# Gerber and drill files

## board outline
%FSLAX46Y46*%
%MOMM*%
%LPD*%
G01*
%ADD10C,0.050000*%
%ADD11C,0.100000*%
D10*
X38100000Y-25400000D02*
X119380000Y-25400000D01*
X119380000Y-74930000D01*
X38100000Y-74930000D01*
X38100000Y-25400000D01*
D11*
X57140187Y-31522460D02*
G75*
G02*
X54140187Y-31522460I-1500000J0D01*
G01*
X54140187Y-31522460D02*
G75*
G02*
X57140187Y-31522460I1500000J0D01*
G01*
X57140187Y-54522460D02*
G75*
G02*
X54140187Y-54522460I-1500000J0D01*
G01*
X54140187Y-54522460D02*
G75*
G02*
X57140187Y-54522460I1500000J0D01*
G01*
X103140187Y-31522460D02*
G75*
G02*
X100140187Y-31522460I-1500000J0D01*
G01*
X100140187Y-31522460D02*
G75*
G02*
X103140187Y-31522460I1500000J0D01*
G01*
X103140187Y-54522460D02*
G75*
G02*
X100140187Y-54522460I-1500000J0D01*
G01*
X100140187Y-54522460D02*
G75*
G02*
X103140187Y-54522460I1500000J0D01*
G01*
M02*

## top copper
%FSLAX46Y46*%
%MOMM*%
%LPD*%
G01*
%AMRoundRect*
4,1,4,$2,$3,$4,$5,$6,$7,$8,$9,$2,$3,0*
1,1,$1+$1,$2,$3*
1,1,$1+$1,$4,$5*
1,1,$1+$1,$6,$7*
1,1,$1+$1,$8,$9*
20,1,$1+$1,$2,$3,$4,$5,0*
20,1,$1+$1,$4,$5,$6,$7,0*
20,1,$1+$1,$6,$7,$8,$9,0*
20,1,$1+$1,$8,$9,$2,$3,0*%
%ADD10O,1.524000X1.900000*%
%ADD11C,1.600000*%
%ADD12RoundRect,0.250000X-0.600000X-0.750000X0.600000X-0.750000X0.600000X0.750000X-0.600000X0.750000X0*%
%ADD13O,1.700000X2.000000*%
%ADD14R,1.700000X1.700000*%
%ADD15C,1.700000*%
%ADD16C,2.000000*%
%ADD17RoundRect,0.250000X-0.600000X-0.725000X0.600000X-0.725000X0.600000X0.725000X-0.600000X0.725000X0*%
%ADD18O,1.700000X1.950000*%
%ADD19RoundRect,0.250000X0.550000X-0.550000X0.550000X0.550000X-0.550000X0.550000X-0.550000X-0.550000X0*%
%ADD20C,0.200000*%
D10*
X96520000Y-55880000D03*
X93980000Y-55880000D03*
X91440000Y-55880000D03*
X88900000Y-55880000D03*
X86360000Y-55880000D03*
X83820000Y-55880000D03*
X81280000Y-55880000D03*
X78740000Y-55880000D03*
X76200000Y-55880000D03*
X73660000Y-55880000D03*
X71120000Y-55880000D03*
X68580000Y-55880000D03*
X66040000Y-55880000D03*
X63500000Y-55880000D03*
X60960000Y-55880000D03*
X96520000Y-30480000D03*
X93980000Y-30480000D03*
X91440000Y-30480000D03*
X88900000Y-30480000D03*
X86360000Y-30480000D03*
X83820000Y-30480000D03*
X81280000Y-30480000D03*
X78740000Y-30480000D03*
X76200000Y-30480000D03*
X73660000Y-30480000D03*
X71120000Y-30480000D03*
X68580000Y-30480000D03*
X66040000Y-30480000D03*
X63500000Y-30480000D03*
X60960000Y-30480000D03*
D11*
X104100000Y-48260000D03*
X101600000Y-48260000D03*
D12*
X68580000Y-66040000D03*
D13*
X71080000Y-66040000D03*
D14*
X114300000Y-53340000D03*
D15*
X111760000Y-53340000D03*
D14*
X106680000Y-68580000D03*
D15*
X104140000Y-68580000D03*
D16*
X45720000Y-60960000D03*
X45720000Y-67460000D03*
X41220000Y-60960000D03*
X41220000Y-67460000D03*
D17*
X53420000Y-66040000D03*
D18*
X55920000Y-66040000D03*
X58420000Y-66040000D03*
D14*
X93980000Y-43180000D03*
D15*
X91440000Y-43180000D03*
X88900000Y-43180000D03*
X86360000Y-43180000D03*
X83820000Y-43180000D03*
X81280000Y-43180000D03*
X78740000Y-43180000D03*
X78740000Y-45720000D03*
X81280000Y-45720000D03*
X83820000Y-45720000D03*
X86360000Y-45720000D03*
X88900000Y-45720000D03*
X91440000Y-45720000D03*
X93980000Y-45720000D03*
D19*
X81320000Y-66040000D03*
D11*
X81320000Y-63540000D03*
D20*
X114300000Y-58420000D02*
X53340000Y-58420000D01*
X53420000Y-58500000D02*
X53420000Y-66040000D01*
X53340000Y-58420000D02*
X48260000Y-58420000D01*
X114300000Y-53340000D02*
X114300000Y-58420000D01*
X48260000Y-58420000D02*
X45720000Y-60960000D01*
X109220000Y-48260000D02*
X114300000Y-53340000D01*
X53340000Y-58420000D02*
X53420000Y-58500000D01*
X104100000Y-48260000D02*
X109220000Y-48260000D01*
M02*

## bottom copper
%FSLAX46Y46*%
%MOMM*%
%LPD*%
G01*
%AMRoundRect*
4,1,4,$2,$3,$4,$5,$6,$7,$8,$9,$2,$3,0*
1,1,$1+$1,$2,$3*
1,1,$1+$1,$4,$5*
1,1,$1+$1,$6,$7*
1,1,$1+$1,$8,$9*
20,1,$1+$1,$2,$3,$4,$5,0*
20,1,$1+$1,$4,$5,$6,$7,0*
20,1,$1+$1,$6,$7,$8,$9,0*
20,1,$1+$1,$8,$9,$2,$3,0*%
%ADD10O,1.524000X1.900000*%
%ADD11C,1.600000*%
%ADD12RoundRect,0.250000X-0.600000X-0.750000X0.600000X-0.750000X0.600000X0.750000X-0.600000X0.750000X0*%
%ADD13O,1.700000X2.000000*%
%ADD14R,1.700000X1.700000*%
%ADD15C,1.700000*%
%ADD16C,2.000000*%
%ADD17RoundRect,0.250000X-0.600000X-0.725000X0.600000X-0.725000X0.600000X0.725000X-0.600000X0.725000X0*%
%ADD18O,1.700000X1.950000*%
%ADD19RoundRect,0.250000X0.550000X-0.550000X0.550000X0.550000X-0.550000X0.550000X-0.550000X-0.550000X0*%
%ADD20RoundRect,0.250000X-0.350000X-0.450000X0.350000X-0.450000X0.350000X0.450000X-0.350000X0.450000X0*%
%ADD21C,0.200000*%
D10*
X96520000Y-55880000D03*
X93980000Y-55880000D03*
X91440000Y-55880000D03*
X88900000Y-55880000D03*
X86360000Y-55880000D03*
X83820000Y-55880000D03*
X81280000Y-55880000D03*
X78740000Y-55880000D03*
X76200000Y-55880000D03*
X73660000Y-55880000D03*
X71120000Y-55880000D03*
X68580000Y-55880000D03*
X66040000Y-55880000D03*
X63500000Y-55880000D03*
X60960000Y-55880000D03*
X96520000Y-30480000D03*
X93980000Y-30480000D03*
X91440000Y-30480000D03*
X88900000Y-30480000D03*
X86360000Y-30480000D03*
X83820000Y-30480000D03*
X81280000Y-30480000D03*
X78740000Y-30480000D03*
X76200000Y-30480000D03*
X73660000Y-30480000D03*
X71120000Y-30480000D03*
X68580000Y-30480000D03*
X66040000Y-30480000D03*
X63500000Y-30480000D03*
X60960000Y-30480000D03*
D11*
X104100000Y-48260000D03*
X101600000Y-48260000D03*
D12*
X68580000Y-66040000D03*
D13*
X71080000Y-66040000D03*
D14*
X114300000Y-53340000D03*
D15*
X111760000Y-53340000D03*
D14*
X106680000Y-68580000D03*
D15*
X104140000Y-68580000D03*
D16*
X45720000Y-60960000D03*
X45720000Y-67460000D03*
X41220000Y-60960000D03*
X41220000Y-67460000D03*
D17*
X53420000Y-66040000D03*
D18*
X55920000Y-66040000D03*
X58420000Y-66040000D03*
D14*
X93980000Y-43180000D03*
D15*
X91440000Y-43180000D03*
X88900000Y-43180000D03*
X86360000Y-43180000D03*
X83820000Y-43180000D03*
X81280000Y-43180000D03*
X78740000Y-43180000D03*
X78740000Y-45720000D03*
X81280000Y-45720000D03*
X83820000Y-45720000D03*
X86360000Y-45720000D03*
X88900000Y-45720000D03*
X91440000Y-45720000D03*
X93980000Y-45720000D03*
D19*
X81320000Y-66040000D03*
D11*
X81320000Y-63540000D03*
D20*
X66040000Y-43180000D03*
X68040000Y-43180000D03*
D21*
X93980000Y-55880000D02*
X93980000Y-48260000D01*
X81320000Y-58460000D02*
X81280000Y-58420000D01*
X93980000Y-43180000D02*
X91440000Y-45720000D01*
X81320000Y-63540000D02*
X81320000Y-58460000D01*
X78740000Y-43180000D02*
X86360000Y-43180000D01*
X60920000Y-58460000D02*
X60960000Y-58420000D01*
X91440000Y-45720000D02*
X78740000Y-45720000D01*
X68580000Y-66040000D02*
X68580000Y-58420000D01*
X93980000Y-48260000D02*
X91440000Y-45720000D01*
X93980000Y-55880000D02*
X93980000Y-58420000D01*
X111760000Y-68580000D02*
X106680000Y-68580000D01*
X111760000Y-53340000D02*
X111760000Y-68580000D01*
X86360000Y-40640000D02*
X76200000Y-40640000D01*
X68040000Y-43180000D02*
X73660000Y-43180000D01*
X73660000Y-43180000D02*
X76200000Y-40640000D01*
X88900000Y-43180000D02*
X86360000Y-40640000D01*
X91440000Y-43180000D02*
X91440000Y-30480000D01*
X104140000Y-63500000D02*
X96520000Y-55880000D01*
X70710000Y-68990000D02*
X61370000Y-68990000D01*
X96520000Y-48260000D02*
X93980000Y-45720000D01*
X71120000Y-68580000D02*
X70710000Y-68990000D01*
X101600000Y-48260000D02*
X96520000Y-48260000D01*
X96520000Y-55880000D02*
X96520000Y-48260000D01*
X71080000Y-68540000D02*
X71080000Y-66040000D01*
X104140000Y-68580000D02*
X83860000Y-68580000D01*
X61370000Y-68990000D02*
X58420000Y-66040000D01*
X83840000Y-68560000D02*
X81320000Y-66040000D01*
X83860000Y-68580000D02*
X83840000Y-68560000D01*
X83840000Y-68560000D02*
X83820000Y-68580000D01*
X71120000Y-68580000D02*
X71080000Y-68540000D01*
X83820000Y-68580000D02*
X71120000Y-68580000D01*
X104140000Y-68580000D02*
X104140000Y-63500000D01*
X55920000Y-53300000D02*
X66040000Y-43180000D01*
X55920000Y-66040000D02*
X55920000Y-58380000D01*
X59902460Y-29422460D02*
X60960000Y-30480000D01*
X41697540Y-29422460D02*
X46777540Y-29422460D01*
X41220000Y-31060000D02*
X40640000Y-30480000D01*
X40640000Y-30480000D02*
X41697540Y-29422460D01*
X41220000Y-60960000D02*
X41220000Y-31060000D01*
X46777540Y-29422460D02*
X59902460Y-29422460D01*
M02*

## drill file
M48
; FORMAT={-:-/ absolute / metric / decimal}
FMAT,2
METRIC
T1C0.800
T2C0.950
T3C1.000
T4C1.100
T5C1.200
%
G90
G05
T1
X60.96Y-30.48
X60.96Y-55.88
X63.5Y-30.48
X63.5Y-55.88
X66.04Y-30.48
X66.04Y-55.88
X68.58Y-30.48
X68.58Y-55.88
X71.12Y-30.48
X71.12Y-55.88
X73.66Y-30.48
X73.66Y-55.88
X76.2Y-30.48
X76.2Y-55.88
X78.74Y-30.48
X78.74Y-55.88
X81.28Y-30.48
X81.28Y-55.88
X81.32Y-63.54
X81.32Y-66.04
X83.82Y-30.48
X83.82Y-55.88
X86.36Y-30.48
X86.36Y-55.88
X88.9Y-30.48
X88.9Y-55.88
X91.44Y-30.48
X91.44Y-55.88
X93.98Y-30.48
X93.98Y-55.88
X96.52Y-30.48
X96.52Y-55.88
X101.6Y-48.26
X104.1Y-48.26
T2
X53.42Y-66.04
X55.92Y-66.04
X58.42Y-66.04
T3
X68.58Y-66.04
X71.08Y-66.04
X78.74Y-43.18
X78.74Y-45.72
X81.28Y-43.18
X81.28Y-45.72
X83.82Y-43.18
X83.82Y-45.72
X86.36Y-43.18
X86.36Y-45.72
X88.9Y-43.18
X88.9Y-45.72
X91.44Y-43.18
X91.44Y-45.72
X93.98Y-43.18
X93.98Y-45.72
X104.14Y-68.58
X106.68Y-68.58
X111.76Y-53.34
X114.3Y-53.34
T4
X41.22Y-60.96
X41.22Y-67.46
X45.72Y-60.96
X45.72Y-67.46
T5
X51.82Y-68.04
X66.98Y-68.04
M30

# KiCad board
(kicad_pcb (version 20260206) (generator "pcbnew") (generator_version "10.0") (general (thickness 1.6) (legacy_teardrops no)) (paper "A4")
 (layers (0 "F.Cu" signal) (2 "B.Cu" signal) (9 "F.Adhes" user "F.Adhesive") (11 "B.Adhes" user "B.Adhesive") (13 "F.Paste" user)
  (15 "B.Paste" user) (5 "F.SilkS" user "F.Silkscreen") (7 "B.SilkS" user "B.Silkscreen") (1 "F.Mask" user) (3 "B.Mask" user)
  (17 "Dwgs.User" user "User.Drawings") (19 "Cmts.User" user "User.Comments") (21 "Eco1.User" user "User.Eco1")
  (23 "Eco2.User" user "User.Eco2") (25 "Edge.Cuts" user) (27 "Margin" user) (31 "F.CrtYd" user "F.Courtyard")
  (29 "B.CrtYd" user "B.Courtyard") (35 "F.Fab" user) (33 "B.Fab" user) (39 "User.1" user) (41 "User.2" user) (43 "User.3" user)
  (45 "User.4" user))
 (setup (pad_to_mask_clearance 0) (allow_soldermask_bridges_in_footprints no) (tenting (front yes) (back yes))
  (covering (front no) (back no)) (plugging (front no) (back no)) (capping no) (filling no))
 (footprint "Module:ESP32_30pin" (layer "F.Cu") (at 79.500187 43.95246 90)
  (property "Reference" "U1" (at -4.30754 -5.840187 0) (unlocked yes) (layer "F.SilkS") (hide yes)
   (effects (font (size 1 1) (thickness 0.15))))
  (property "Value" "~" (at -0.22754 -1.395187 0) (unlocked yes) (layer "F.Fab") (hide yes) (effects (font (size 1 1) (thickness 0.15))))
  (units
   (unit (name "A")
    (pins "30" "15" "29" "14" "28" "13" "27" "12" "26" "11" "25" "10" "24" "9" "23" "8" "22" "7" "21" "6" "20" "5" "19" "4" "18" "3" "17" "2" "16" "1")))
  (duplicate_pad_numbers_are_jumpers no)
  (fp_circle (center 12.43 -23.86) (end 12.43 -22.36) (stroke (width 0.1) (type default)) (fill no) (layer "Edge.Cuts"))
  (fp_circle (center -10.57 -23.86) (end -10.57 -22.36) (stroke (width 0.1) (type default)) (fill no) (layer "Edge.Cuts"))
  (fp_circle (center 12.43 22.14) (end 12.43 23.64) (stroke (width 0.1) (type default)) (fill no) (layer "Edge.Cuts"))
  (fp_circle (center -10.57 22.14) (end -10.57 23.64) (stroke (width 0.1) (type default)) (fill no) (layer "Edge.Cuts"))
  (pad "1" thru_hole oval (at -11.92754 17.019813) (size 1.524 1.9) (drill 0.8) (layers "*.Cu" "*.Mask") (remove_unused_layers no)
   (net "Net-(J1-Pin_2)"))
  (pad "2" thru_hole oval (at -11.92754 14.479813) (size 1.524 1.9) (drill 0.8) (layers "*.Cu" "*.Mask") (remove_unused_layers no)
   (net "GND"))
  (pad "3" thru_hole oval (at -11.92754 11.939813) (size 1.524 1.9) (drill 0.8) (layers "*.Cu" "*.Mask") (remove_unused_layers no)
   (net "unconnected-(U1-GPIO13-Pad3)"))
  (pad "4" thru_hole oval (at -11.92754 9.399813) (size 1.524 1.9) (drill 0.8) (layers "*.Cu" "*.Mask") (remove_unused_layers no)
   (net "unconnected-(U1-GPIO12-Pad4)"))
  (pad "5" thru_hole oval (at -11.92754 6.859813) (size 1.524 1.9) (drill 0.8) (layers "*.Cu" "*.Mask") (remove_unused_layers no)
   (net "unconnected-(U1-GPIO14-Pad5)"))
  (pad "6" thru_hole oval (at -11.92754 4.319813) (size 1.524 1.9) (drill 0.8) (layers "*.Cu" "*.Mask") (remove_unused_layers no)
   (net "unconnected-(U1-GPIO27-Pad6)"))
  (pad "7" thru_hole oval (at -11.92754 1.779813) (size 1.524 1.9) (drill 0.8) (layers "*.Cu" "*.Mask") (remove_unused_layers no)
   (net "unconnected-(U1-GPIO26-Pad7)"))
  (pad "8" thru_hole oval (at -11.92754 -0.760187) (size 1.524 1.9) (drill 0.8) (layers "*.Cu" "*.Mask") (remove_unused_layers no)
   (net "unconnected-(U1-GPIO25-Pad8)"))
  (pad "9" thru_hole oval (at -11.92754 -3.300187) (size 1.524 1.9) (drill 0.8) (layers "*.Cu" "*.Mask") (remove_unused_layers no)
   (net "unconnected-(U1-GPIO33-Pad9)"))
  (pad "10" thru_hole oval (at -11.92754 -5.840187) (size 1.524 1.9) (drill 0.8) (layers "*.Cu" "*.Mask") (remove_unused_layers no)
   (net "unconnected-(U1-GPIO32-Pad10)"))
  (pad "11" thru_hole oval (at -11.92754 -8.380187) (size 1.524 1.9) (drill 0.8) (layers "*.Cu" "*.Mask") (remove_unused_layers no)
   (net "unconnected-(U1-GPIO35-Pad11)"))
  (pad "12" thru_hole oval (at -11.92754 -10.920187) (size 1.524 1.9) (drill 0.8) (layers "*.Cu" "*.Mask") (remove_unused_layers no)
   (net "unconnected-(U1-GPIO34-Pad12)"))
  (pad "13" thru_hole oval (at -11.92754 -13.460187) (size 1.524 1.9) (drill 0.8) (layers "*.Cu" "*.Mask") (remove_unused_layers no)
   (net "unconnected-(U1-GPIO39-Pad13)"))
  (pad "14" thru_hole oval (at -11.92754 -16.000187) (size 1.524 1.9) (drill 0.8) (layers "*.Cu" "*.Mask") (remove_unused_layers no)
   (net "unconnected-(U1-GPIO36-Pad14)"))
  (pad "15" thru_hole oval (at -11.92754 -18.540187) (size 1.524 1.9) (drill 0.8) (layers "*.Cu" "*.Mask") (remove_unused_layers no)
   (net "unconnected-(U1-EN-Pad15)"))
  (pad "16" thru_hole oval (at 13.47246 17.019813) (size 1.524 1.9) (drill 0.8) (layers "*.Cu" "*.Mask") (remove_unused_layers no)
   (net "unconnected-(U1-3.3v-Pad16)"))
  (pad "17" thru_hole oval (at 13.47246 14.479813) (size 1.524 1.9) (drill 0.8) (layers "*.Cu" "*.Mask") (remove_unused_layers no)
   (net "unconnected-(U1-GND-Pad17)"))
  (pad "18" thru_hole oval (at 13.47246 11.939813) (size 1.524 1.9) (drill 0.8) (layers "*.Cu" "*.Mask") (remove_unused_layers no)
   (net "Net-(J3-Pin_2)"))
  (pad "19" thru_hole oval (at 13.47246 9.399813) (size 1.524 1.9) (drill 0.8) (layers "*.Cu" "*.Mask") (remove_unused_layers no)
   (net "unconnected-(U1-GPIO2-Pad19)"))
  (pad "20" thru_hole oval (at 13.47246 6.859813) (size 1.524 1.9) (drill 0.8) (layers "*.Cu" "*.Mask" "Dwgs.User")
   (remove_unused_layers no) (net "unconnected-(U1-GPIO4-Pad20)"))
  (pad "21" thru_hole oval (at 13.47246 4.319813) (size 1.524 1.9) (drill 0.8) (layers "*.Cu" "*.Mask") (remove_unused_layers no)
   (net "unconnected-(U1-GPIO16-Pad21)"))
  (pad "22" thru_hole oval (at 13.47246 1.779813) (size 1.524 1.9) (drill 0.8) (layers "*.Cu" "*.Mask") (remove_unused_layers no)
   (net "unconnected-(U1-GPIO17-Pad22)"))
  (pad "23" thru_hole oval (at 13.47246 -0.760187) (size 1.524 1.9) (drill 0.8) (layers "*.Cu" "*.Mask") (remove_unused_layers no)
   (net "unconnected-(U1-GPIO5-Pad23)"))
  (pad "24" thru_hole oval (at 13.47246 -3.300187) (size 1.524 1.9) (drill 0.8) (layers "*.Cu" "*.Mask") (remove_unused_layers no)
   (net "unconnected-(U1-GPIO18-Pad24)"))
  (pad "25" thru_hole oval (at 13.47246 -5.840187) (size 1.524 1.9) (drill 0.8) (layers "*.Cu" "*.Mask") (remove_unused_layers no)
   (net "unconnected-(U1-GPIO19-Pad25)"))
  (pad "26" thru_hole oval (at 13.47246 -8.380187) (size 1.524 1.9) (drill 0.8) (layers "*.Cu" "*.Mask") (remove_unused_layers no)
   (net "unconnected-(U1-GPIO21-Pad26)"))
  (pad "27" thru_hole oval (at 13.47246 -10.920187) (size 1.524 1.9) (drill 0.8) (layers "*.Cu" "*.Mask") (remove_unused_layers no)
   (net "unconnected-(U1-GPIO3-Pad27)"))
  (pad "28" thru_hole oval (at 13.47246 -13.460187) (size 1.524 1.9) (drill 0.8) (layers "*.Cu" "*.Mask") (remove_unused_layers no)
   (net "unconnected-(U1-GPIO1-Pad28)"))
  (pad "29" thru_hole oval (at 13.47246 -16.000187) (size 1.524 1.9) (drill 0.8) (layers "*.Cu" "*.Mask") (remove_unused_layers no)
   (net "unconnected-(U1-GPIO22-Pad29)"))
  (pad "30" thru_hole oval (at 13.47246 -18.540187) (size 1.524 1.9) (drill 0.8) (layers "*.Cu" "*.Mask") (remove_unused_layers no)
   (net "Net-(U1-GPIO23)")))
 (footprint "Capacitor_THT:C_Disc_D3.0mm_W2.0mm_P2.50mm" (layer "F.Cu") (at 104.1 48.26 180)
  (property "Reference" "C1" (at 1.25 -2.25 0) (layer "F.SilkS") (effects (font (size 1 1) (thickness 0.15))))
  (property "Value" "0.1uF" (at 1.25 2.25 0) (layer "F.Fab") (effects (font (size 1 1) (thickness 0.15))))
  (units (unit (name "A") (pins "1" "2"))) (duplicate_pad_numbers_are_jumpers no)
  (pad "1" thru_hole circle (at 0 0 180) (size 1.6 1.6) (drill 0.8) (layers "*.Cu" "*.Mask") (remove_unused_layers no) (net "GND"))
  (pad "2" thru_hole circle (at 2.5 0 180) (size 1.6 1.6) (drill 0.8) (layers "*.Cu" "*.Mask") (remove_unused_layers no)
   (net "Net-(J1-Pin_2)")))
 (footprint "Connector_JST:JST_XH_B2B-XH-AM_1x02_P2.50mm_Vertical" (layer "F.Cu") (at 68.58 66.04)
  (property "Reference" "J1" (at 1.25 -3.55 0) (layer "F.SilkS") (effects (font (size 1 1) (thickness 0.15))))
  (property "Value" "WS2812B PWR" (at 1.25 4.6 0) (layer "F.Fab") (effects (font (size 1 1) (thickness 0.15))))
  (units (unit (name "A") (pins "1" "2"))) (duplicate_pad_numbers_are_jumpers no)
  (pad "" np_thru_hole circle (at -1.6 2) (size 1.2 1.2) (drill 1.2) (layers "*.Cu" "*.Mask"))
  (pad "1" thru_hole roundrect (at 0 0) (size 1.7 2) (drill 1) (layers "*.Cu" "*.Mask") (remove_unused_layers no)
   (roundrect_rratio 0.147059) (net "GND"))
  (pad "2" thru_hole oval (at 2.5 0) (size 1.7 2) (drill 1) (layers "*.Cu" "*.Mask") (remove_unused_layers no) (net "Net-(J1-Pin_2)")))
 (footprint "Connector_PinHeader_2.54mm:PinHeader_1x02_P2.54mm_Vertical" (layer "F.Cu") (at 114.3 53.34 -90)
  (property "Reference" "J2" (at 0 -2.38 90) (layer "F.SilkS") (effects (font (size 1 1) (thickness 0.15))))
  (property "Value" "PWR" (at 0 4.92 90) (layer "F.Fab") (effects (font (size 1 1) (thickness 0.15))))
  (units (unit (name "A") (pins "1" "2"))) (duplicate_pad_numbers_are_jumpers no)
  (pad "1" thru_hole rect (at 0 0 270) (size 1.7 1.7) (drill 1) (layers "*.Cu" "*.Mask") (remove_unused_layers no) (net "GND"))
  (pad "2" thru_hole circle (at 0 2.54 270) (size 1.7 1.7) (drill 1) (layers "*.Cu" "*.Mask") (remove_unused_layers no) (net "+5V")))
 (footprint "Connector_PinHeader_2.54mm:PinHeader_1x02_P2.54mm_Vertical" (layer "F.Cu") (at 106.68 68.58 -90)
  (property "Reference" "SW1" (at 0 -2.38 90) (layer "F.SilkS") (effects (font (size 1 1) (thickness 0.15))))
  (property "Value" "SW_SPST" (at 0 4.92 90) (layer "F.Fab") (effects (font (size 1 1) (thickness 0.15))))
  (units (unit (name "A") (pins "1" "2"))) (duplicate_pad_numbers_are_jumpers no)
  (pad "1" thru_hole rect (at 0 0 270) (size 1.7 1.7) (drill 1) (layers "*.Cu" "*.Mask") (remove_unused_layers no) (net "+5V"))
  (pad "2" thru_hole circle (at 0 2.54 270) (size 1.7 1.7) (drill 1) (layers "*.Cu" "*.Mask") (remove_unused_layers no)
   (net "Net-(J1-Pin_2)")))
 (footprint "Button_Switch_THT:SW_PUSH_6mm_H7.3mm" (layer "F.Cu") (at 45.72 60.96 -90)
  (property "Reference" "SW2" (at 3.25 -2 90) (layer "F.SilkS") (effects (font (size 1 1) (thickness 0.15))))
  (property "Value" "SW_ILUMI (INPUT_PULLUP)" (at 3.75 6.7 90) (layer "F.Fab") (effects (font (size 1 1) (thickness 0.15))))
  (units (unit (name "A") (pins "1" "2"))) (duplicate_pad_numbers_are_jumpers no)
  (pad "1" thru_hole circle (at 0 0) (size 2 2) (drill 1.1) (layers "*.Cu" "*.Mask") (remove_unused_layers no) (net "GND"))
  (pad "1" thru_hole circle (at 6.5 0) (size 2 2) (drill 1.1) (layers "*.Cu" "*.Mask") (remove_unused_layers no) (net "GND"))
  (pad "2" thru_hole circle (at 0 4.5) (size 2 2) (drill 1.1) (layers "*.Cu" "*.Mask") (remove_unused_layers no) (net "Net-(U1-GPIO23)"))
  (pad "2" thru_hole circle (at 6.5 4.5) (size 2 2) (drill 1.1) (layers "*.Cu" "*.Mask") (remove_unused_layers no) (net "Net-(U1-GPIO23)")))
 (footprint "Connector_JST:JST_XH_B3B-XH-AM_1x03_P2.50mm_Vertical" (layer "F.Cu") (at 53.42 66.04)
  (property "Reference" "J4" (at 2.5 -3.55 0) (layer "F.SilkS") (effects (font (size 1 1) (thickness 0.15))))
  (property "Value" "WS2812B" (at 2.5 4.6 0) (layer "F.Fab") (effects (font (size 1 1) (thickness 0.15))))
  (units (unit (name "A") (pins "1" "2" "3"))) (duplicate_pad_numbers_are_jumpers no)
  (pad "" np_thru_hole circle (at -1.6 2) (size 1.2 1.2) (drill 1.2) (layers "*.Cu" "*.Mask"))
  (pad "1" thru_hole roundrect (at 0 0) (size 1.7 1.95) (drill 0.95) (layers "*.Cu" "*.Mask") (remove_unused_layers no)
   (roundrect_rratio 0.147059) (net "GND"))
  (pad "2" thru_hole oval (at 2.5 0) (size 1.7 1.95) (drill 0.95) (layers "*.Cu" "*.Mask") (remove_unused_layers no) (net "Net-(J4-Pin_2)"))
  (pad "3" thru_hole oval (at 5 0) (size 1.7 1.95) (drill 0.95) (layers "*.Cu" "*.Mask") (remove_unused_layers no) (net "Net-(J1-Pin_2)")))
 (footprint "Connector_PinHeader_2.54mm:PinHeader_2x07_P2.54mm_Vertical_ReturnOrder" (layer "F.Cu") (at 93.98 43.18 -90)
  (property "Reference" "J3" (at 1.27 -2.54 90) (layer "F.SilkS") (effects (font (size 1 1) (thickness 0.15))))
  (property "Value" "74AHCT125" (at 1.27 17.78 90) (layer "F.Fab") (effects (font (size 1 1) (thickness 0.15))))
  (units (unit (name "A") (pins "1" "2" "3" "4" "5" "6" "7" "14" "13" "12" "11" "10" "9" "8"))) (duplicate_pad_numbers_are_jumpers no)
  (pad "1" thru_hole rect (at 0 0 270) (size 1.7 1.7) (drill 1) (layers "*.Cu" "*.Mask") (remove_unused_layers no) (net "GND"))
  (pad "2" thru_hole circle (at 0 2.54 270) (size 1.7 1.7) (drill 1) (layers "*.Cu" "*.Mask") (remove_unused_layers no)
   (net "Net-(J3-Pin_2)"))
  (pad "3" thru_hole circle (at 0 5.08 270) (size 1.7 1.7) (drill 1) (layers "*.Cu" "*.Mask") (remove_unused_layers no)
   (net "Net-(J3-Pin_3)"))
  (pad "4" thru_hole circle (at 0 7.62 270) (size 1.7 1.7) (drill 1) (layers "*.Cu" "*.Mask") (remove_unused_layers no) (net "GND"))
  (pad "5" thru_hole circle (at 0 10.16 270) (size 1.7 1.7) (drill 1) (layers "*.Cu" "*.Mask") (remove_unused_layers no) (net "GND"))
  (pad "6" thru_hole circle (at 0 12.7 270) (size 1.7 1.7) (drill 1) (layers "*.Cu" "*.Mask") (remove_unused_layers no) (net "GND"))
  (pad "7" thru_hole circle (at 0 15.24 270) (size 1.7 1.7) (drill 1) (layers "*.Cu" "*.Mask") (remove_unused_layers no) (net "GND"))
  (pad "8" thru_hole circle (at 2.54 15.24 270) (size 1.7 1.7) (drill 1) (layers "*.Cu" "*.Mask") (remove_unused_layers no) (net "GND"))
  (pad "9" thru_hole circle (at 2.54 12.7 270) (size 1.7 1.7) (drill 1) (layers "*.Cu" "*.Mask") (remove_unused_layers no) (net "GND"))
  (pad "10" thru_hole circle (at 2.54 10.16 270) (size 1.7 1.7) (drill 1) (layers "*.Cu" "*.Mask") (remove_unused_layers no) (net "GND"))
  (pad "11" thru_hole circle (at 2.54 7.62 270) (size 1.7 1.7) (drill 1) (layers "*.Cu" "*.Mask") (remove_unused_layers no) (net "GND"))
  (pad "12" thru_hole circle (at 2.54 5.08 270) (size 1.7 1.7) (drill 1) (layers "*.Cu" "*.Mask") (remove_unused_layers no) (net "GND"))
  (pad "13" thru_hole circle (at 2.54 2.54 270) (size 1.7 1.7) (drill 1) (layers "*.Cu" "*.Mask") (remove_unused_layers no) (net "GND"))
  (pad "14" thru_hole circle (at 2.54 0 270) (size 1.7 1.7) (drill 1) (layers "*.Cu" "*.Mask") (remove_unused_layers no)
   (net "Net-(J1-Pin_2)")))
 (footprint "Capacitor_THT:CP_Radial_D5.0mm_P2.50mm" (layer "F.Cu") (at 81.32 66.04 90)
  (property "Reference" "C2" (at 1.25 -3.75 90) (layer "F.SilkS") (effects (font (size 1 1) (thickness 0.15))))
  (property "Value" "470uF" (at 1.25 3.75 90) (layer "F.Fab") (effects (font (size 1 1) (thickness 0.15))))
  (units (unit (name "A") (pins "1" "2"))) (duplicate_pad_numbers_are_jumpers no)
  (pad "1" thru_hole roundrect (at 0 0 90) (size 1.6 1.6) (drill 0.8) (layers "*.Cu" "*.Mask") (remove_unused_layers no)
   (roundrect_rratio 0.15625) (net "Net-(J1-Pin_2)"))
  (pad "2" thru_hole circle (at 2.5 0 90) (size 1.6 1.6) (drill 0.8) (layers "*.Cu" "*.Mask") (remove_unused_layers no) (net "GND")))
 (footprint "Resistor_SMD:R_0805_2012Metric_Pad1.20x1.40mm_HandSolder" (layer "B.Cu") (at 67.04 43.18)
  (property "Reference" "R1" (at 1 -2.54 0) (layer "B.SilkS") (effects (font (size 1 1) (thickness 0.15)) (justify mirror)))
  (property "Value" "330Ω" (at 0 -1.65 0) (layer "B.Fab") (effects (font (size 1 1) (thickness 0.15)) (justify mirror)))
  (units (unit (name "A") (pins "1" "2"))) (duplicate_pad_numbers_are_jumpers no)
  (pad "1" smd roundrect (at -1 0) (size 1.2 1.4) (layers "B.Cu" "B.Mask" "B.Paste") (roundrect_rratio 0.208333) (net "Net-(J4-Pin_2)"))
  (pad "2" smd roundrect (at 1 0) (size 1.2 1.4) (layers "B.Cu" "B.Mask" "B.Paste") (roundrect_rratio 0.208333) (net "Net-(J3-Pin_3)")))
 (gr_rect (start 38.1 25.4) (end 119.38 74.93) (stroke (width 0.05) (type default)) (fill no) (layer "Edge.Cuts"))
 (segment (start 114.3 58.42) (end 53.34 58.42) (width 0.2) (layer "F.Cu") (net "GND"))
 (segment (start 53.42 58.5) (end 53.42 66.04) (width 0.2) (layer "F.Cu") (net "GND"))
 (segment (start 53.34 58.42) (end 48.26 58.42) (width 0.2) (layer "F.Cu") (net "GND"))
 (segment (start 114.3 53.34) (end 114.3 58.42) (width 0.2) (layer "F.Cu") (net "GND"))
 (segment (start 48.26 58.42) (end 45.72 60.96) (width 0.2) (layer "F.Cu") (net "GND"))
 (segment (start 109.22 48.26) (end 114.3 53.34) (width 0.2) (layer "F.Cu") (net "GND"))
 (segment (start 53.34 58.42) (end 53.42 58.5) (width 0.2) (layer "F.Cu") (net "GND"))
 (segment (start 104.1 48.26) (end 109.22 48.26) (width 0.2) (layer "F.Cu") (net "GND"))
 (segment (start 93.98 55.88) (end 93.98 48.26) (width 0.2) (layer "B.Cu") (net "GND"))
 (segment (start 81.32 58.46) (end 81.28 58.42) (width 0.2) (layer "B.Cu") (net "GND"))
 (segment (start 93.98 43.18) (end 91.44 45.72) (width 0.2) (layer "B.Cu") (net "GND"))
 (segment (start 81.32 63.54) (end 81.32 58.46) (width 0.2) (layer "B.Cu") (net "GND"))
 (segment (start 78.74 43.18) (end 86.36 43.18) (width 0.2) (layer "B.Cu") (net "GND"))
 (segment (start 60.92 58.46) (end 60.96 58.42) (width 0.2) (layer "B.Cu") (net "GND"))
 (segment (start 91.44 45.72) (end 78.74 45.72) (width 0.2) (layer "B.Cu") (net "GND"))
 (segment (start 68.58 66.04) (end 68.58 58.42) (width 0.2) (layer "B.Cu") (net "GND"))
 (segment (start 93.98 48.26) (end 91.44 45.72) (width 0.2) (layer "B.Cu") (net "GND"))
 (segment (start 93.98 55.88) (end 93.98 58.42) (width 0.2) (layer "B.Cu") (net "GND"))
 (segment (start 111.76 68.58) (end 106.68 68.58) (width 0.2) (layer "B.Cu") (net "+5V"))
 (segment (start 111.76 53.34) (end 111.76 68.58) (width 0.2) (layer "B.Cu") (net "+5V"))
 (segment (start 86.36 40.64) (end 76.2 40.64) (width 0.2) (layer "B.Cu") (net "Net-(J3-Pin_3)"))
 (segment (start 68.04 43.18) (end 73.66 43.18) (width 0.2) (layer "B.Cu") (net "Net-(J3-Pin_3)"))
 (segment (start 73.66 43.18) (end 76.2 40.64) (width 0.2) (layer "B.Cu") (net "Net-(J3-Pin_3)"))
 (segment (start 88.9 43.18) (end 86.36 40.64) (width 0.2) (layer "B.Cu") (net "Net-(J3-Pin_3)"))
 (segment (start 91.44 43.18) (end 91.44 30.48) (width 0.2) (layer "B.Cu") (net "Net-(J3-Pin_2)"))
 (segment (start 104.14 63.5) (end 96.52 55.88) (width 0.2) (layer "B.Cu") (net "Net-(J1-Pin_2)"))
 (segment (start 70.71 68.99) (end 61.37 68.99) (width 0.2) (layer "B.Cu") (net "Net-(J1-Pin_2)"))
 (segment (start 96.52 48.26) (end 93.98 45.72) (width 0.2) (layer "B.Cu") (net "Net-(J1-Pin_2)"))
 (segment (start 71.12 68.58) (end 70.71 68.99) (width 0.2) (layer "B.Cu") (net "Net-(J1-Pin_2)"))
 (segment (start 101.6 48.26) (end 96.52 48.26) (width 0.2) (layer "B.Cu") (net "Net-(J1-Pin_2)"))
 (segment (start 96.52 55.88) (end 96.52 48.26) (width 0.2) (layer "B.Cu") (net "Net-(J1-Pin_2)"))
 (segment (start 71.08 68.54) (end 71.08 66.04) (width 0.2) (layer "B.Cu") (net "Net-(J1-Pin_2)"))
 (segment (start 104.14 68.58) (end 83.86 68.58) (width 0.2) (layer "B.Cu") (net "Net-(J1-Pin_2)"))
 (segment (start 61.37 68.99) (end 58.42 66.04) (width 0.2) (layer "B.Cu") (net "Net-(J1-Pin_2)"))
 (segment (start 83.84 68.56) (end 81.32 66.04) (width 0.2) (layer "B.Cu") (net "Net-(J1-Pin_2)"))
 (segment (start 83.86 68.58) (end 83.84 68.56) (width 0.2) (layer "B.Cu") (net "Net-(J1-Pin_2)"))
 (segment (start 83.84 68.56) (end 83.82 68.58) (width 0.2) (layer "B.Cu") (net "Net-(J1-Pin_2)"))
 (segment (start 71.12 68.58) (end 71.08 68.54) (width 0.2) (layer "B.Cu") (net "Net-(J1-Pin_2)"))
 (segment (start 83.82 68.58) (end 71.12 68.58) (width 0.2) (layer "B.Cu") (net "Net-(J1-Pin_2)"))
 (segment (start 104.14 68.58) (end 104.14 63.5) (width 0.2) (layer "B.Cu") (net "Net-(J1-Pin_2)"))
 (segment (start 55.92 53.3) (end 66.04 43.18) (width 0.2) (layer "B.Cu") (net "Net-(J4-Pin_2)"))
 (segment (start 55.92 66.04) (end 55.92 58.38) (width 0.2) (layer "B.Cu") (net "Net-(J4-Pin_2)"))
 (segment (start 59.90246 29.42246) (end 60.96 30.48) (width 0.2) (layer "B.Cu") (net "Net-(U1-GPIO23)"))
 (segment (start 41.69754 29.42246) (end 46.77754 29.42246) (width 0.2) (layer "B.Cu") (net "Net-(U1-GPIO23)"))
 (segment (start 41.22 31.06) (end 40.64 30.48) (width 0.2) (layer "B.Cu") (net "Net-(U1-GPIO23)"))
 (segment (start 40.64 30.48) (end 41.69754 29.42246) (width 0.2) (layer "B.Cu") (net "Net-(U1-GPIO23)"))
 (segment (start 41.22 60.96) (end 41.22 31.06) (width 0.2) (layer "B.Cu") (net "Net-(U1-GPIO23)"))
 (segment (start 46.77754 29.42246) (end 59.90246 29.42246) (width 0.2) (layer "B.Cu") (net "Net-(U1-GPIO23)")))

